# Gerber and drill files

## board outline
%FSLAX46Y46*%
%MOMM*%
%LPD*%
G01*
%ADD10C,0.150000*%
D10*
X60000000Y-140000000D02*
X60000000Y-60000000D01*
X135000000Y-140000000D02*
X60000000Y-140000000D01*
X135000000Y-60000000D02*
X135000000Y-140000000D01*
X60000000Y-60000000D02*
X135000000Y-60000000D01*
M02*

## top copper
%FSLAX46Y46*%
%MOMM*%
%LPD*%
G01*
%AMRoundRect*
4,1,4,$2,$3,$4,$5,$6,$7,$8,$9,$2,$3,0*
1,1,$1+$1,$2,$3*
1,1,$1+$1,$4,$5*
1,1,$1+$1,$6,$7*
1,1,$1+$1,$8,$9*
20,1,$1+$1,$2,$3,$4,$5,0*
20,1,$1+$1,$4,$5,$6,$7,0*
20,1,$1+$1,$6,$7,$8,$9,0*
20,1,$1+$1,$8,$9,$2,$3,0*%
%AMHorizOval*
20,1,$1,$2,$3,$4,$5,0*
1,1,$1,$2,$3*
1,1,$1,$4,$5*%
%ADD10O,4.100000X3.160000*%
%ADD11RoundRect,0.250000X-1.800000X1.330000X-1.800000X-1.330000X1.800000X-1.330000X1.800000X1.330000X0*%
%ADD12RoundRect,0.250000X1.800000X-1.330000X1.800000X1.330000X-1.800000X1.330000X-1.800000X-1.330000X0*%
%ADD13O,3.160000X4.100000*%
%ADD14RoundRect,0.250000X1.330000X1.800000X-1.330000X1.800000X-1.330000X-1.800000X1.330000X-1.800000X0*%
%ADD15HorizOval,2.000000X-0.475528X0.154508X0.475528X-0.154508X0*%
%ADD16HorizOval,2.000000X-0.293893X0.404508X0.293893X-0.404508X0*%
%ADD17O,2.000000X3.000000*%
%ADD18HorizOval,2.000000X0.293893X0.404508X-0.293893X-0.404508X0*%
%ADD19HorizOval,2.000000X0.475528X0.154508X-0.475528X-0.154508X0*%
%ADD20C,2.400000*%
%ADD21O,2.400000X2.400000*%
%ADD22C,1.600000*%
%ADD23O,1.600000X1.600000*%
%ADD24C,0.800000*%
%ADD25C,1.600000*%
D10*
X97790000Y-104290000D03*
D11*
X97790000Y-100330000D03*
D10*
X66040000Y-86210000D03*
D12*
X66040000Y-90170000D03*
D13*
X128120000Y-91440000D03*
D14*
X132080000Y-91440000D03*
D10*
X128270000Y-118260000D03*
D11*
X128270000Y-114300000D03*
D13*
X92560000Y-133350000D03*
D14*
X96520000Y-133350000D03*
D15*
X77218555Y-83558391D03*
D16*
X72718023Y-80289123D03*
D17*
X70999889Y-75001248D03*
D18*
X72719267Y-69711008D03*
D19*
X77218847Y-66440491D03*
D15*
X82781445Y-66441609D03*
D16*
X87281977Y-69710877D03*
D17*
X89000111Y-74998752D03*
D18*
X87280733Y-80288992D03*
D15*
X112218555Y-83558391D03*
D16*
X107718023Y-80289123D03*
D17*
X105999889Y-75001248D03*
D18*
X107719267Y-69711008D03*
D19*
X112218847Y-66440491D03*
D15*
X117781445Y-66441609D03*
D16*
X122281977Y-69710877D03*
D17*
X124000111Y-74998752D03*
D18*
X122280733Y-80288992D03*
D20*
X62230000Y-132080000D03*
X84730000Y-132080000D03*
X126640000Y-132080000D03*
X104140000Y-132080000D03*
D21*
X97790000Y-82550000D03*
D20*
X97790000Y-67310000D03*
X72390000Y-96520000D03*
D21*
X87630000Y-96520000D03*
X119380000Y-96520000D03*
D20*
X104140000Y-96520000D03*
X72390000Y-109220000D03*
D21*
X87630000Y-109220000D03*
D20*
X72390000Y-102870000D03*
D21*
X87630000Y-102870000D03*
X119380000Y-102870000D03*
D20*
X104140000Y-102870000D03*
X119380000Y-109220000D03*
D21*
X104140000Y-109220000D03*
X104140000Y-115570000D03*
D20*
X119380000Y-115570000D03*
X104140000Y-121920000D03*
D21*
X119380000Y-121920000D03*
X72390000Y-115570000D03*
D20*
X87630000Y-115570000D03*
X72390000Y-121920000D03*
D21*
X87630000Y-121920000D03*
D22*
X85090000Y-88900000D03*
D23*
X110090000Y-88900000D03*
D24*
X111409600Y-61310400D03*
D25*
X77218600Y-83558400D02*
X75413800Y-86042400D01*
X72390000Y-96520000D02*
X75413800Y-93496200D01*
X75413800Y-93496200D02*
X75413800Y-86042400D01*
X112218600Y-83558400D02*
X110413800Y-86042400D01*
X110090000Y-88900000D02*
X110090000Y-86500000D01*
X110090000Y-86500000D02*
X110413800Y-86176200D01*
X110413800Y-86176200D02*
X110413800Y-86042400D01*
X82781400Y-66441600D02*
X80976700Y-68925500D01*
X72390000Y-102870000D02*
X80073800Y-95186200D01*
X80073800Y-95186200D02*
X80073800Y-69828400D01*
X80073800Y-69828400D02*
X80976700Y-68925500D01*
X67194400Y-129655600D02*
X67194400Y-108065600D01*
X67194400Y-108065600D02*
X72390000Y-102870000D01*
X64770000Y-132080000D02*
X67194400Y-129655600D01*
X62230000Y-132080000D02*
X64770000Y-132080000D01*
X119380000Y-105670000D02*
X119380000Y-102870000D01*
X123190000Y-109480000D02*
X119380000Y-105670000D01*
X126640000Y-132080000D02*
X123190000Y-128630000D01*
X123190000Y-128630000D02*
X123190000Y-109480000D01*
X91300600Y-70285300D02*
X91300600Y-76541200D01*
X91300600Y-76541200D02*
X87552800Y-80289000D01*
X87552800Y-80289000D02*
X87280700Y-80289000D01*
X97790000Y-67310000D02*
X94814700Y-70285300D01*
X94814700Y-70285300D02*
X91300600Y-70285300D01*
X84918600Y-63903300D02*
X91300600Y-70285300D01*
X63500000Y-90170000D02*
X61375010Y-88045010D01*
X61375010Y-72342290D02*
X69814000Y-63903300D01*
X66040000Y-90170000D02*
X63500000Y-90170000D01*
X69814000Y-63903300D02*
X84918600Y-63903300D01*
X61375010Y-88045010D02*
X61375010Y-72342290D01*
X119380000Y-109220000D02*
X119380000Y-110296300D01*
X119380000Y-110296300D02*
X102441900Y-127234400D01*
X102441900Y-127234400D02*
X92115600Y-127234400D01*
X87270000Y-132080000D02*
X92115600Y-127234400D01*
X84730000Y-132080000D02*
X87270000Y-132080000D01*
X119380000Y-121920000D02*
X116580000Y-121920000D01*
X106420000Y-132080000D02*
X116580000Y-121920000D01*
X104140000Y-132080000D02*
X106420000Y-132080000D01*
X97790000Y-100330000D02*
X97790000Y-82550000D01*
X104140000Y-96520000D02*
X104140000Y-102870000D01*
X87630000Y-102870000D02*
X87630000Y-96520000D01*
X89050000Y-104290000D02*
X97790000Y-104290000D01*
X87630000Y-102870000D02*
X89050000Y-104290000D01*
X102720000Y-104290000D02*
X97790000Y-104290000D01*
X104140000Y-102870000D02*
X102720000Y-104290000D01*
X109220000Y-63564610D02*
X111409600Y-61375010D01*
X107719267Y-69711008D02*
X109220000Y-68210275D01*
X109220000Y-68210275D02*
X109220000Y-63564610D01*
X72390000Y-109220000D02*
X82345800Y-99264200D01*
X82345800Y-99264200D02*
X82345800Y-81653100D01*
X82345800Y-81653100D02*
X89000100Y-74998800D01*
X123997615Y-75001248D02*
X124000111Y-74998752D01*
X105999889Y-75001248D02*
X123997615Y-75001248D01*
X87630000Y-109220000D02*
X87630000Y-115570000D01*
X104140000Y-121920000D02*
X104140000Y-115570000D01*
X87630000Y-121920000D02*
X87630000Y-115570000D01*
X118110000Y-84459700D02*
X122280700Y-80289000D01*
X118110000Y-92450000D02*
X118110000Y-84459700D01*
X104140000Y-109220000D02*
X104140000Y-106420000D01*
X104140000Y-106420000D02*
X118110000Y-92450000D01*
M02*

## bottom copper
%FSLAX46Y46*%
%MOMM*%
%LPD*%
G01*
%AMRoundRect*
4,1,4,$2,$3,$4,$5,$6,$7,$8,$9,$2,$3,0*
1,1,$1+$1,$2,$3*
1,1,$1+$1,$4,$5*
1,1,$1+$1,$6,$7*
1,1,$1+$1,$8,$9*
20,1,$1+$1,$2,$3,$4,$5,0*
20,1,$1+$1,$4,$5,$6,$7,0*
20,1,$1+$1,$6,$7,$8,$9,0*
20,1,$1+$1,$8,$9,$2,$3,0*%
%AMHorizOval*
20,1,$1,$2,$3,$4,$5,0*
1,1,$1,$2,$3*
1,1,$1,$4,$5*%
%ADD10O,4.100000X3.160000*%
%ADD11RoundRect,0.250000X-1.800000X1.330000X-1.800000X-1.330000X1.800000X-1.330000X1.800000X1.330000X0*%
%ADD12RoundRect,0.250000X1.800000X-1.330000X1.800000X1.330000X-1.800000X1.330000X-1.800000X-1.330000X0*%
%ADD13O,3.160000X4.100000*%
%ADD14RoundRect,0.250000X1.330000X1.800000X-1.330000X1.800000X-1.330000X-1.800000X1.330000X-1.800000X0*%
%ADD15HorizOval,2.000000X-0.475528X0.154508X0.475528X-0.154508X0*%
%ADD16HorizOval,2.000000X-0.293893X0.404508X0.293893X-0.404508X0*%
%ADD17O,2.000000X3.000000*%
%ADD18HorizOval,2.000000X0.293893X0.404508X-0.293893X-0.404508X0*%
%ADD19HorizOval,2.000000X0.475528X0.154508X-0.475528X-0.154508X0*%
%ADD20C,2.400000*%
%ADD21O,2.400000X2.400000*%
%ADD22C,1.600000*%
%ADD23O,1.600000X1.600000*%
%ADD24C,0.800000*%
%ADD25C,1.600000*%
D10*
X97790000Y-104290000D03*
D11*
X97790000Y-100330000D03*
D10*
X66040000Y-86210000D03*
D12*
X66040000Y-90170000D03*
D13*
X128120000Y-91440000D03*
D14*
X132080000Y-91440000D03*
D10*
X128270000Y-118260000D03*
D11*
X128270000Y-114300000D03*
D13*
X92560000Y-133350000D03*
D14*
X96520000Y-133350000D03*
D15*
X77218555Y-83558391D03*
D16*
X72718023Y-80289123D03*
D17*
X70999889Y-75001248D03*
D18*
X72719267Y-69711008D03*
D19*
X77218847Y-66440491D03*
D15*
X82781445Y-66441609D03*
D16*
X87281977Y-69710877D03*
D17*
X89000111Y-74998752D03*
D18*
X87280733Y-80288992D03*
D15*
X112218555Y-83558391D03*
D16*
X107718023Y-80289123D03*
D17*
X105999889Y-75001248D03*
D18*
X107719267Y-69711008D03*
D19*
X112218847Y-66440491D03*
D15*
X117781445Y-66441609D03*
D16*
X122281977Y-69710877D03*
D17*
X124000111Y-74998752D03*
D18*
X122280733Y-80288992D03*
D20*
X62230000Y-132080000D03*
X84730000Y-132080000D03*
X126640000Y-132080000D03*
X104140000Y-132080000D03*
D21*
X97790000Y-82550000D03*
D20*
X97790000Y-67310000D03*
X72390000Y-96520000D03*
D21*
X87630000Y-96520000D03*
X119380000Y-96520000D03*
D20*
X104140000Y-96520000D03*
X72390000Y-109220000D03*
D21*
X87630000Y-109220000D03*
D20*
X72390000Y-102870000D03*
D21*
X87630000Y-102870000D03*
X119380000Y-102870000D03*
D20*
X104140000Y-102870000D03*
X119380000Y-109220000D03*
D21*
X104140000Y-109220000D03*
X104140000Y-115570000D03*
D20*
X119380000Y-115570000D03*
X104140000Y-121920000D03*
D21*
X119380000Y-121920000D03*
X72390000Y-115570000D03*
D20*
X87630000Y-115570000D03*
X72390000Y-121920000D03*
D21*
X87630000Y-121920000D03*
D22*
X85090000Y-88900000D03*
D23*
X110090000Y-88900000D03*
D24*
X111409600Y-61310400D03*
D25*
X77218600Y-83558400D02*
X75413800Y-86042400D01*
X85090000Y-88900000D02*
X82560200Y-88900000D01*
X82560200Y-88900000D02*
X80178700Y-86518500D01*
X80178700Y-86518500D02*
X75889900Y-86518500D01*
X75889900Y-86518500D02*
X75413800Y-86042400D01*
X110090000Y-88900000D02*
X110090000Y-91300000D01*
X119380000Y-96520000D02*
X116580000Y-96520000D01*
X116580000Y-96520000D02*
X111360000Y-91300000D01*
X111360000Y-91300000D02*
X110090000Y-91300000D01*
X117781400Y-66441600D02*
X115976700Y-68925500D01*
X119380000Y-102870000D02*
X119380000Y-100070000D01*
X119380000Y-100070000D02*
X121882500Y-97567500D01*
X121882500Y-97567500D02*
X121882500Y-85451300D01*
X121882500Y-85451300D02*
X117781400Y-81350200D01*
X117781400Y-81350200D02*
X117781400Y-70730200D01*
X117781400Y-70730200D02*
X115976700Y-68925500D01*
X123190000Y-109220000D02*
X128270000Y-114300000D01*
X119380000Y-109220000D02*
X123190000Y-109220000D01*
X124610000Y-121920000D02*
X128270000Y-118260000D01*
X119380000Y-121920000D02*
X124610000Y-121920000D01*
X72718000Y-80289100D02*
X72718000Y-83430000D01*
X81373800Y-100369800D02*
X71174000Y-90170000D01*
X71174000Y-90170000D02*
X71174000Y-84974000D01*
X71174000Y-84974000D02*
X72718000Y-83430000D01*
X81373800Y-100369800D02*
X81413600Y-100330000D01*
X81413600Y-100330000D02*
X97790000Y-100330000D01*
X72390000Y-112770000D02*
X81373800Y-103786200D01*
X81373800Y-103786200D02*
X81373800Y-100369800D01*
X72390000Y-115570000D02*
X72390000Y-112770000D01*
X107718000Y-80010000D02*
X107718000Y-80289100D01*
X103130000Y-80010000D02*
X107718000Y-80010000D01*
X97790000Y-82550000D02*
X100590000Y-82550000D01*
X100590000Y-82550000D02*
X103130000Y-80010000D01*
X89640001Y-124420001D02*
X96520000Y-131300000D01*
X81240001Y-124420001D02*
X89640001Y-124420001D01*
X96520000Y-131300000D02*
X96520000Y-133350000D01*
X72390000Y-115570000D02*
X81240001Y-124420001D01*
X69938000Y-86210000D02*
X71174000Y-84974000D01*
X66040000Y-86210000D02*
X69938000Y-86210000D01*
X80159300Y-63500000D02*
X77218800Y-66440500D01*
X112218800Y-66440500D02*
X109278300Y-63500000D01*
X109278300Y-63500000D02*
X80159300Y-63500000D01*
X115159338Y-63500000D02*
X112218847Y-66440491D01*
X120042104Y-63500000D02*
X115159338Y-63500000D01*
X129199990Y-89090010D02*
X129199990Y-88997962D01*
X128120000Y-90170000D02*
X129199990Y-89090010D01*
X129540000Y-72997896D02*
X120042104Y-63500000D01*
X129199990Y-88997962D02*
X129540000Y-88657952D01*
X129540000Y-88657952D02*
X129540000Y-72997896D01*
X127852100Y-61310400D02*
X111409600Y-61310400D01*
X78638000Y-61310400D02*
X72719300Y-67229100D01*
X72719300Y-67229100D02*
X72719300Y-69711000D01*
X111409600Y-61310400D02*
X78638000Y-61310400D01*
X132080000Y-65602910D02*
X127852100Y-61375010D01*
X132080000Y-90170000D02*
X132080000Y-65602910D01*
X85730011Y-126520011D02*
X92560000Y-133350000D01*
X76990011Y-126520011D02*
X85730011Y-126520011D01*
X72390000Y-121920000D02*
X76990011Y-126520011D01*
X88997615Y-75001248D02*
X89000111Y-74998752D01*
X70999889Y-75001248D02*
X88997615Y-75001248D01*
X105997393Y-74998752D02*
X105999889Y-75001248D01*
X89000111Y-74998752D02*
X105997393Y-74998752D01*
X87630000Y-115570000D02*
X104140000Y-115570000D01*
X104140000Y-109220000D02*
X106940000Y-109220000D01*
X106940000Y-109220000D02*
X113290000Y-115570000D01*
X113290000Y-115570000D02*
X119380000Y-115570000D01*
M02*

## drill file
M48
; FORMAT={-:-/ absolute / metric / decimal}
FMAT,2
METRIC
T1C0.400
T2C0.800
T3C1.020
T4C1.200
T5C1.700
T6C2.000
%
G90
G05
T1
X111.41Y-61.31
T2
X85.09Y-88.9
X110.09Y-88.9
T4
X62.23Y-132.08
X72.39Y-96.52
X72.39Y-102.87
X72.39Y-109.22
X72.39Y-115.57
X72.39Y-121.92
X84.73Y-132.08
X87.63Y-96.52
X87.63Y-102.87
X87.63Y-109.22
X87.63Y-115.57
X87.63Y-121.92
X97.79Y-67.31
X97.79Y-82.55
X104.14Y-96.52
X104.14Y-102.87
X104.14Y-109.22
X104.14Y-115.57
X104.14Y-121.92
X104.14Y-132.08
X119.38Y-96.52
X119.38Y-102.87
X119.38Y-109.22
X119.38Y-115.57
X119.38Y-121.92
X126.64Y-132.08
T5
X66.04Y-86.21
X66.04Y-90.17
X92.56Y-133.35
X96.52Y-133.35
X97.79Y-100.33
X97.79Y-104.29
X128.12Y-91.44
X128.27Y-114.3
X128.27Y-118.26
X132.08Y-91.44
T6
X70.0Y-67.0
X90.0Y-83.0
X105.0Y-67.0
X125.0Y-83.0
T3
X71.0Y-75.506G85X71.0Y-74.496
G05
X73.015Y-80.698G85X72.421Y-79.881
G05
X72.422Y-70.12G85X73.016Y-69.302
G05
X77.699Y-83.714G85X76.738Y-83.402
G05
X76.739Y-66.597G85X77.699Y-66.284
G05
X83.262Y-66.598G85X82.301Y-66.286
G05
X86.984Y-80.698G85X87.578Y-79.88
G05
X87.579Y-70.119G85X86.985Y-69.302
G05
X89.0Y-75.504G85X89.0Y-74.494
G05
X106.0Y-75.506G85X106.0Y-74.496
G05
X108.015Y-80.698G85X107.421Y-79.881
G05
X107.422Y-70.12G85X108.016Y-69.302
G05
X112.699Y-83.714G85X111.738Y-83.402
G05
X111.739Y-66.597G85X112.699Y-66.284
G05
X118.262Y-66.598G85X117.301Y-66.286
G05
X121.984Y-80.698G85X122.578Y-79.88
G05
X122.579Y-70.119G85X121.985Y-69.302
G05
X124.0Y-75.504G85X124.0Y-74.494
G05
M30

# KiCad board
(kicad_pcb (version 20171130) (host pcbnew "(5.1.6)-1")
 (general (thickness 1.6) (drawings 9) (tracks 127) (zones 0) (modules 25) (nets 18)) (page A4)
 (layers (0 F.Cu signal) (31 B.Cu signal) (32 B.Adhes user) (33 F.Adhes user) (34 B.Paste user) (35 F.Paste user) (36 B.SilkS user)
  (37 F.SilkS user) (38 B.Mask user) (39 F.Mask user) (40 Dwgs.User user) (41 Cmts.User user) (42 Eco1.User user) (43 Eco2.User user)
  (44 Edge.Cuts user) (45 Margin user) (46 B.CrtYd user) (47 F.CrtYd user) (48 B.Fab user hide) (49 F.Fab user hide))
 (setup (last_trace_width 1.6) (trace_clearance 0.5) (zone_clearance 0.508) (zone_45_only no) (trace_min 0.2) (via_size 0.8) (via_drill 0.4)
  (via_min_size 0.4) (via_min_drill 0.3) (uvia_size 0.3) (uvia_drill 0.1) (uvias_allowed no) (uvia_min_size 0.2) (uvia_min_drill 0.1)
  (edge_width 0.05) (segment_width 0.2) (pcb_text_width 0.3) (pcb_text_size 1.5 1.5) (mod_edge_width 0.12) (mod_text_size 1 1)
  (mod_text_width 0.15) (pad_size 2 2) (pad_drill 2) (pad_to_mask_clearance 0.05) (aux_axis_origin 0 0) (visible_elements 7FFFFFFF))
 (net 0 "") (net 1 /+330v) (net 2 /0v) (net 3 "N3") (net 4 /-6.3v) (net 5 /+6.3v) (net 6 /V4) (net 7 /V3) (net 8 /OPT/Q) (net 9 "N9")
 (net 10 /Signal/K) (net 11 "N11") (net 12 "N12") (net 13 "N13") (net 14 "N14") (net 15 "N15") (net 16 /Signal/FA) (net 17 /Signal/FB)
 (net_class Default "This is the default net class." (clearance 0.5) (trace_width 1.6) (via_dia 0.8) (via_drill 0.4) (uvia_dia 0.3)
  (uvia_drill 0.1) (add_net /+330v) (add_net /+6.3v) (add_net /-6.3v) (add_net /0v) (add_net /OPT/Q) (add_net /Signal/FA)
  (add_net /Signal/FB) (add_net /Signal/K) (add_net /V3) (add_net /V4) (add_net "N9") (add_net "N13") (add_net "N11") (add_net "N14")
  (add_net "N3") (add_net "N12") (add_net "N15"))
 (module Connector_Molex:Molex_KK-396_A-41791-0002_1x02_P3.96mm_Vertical (layer F.Cu) (at 97.79 100.33 270)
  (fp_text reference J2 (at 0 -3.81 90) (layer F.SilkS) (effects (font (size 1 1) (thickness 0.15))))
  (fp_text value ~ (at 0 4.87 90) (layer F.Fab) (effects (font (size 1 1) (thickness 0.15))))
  (pad 2 thru_hole oval (at 3.96 0 270) (size 3.16 4.1) (drill 1.7) (layers *.Cu *.Mask) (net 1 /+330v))
  (pad 1 thru_hole roundrect (at 0 0 270) (size 3.16 4.1) (drill 1.7) (layers *.Cu *.Mask) (roundrect_rratio 0.079114) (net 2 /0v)))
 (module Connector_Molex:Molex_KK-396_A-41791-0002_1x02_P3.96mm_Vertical (layer F.Cu) (at 66.04 90.17 90)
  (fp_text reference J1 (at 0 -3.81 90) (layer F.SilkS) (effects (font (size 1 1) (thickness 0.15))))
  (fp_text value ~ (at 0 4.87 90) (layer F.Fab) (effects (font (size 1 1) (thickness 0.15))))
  (pad 2 thru_hole oval (at 3.96 0 90) (size 3.16 4.1) (drill 1.7) (layers *.Cu *.Mask) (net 2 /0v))
  (pad 1 thru_hole roundrect (at 0 0 90) (size 3.16 4.1) (drill 1.7) (layers *.Cu *.Mask) (roundrect_rratio 0.079114) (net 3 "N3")))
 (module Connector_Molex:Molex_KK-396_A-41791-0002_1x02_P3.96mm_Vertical (layer F.Cu) (at 132.08 91.44 180)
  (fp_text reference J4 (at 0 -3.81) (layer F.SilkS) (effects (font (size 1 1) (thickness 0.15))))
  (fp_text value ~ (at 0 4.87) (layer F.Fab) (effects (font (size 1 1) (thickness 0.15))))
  (pad 2 thru_hole oval (at 3.96 0 180) (size 3.16 4.1) (drill 1.7) (layers *.Cu *.Mask) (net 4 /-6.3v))
  (pad 1 thru_hole roundrect (at 0 0 180) (size 3.16 4.1) (drill 1.7) (layers *.Cu *.Mask) (roundrect_rratio 0.079114) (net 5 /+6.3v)))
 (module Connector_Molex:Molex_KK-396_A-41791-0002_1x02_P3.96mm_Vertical (layer F.Cu) (at 128.27 114.3 270)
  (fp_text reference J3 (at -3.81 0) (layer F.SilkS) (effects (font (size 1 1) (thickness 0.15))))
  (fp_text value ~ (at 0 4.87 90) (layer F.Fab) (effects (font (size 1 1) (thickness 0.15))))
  (pad 2 thru_hole oval (at 3.96 0 270) (size 3.16 4.1) (drill 1.7) (layers *.Cu *.Mask) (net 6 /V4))
  (pad 1 thru_hole roundrect (at 0 0 270) (size 3.16 4.1) (drill 1.7) (layers *.Cu *.Mask) (roundrect_rratio 0.079114) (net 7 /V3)))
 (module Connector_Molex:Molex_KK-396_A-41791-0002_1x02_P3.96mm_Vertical (layer F.Cu) (at 96.52 133.35 180)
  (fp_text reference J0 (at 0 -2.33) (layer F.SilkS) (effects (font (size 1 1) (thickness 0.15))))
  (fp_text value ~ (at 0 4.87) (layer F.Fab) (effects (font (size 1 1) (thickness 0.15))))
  (pad 2 thru_hole oval (at 3.96 0 180) (size 3.16 4.1) (drill 1.7) (layers *.Cu *.Mask) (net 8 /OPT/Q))
  (pad 1 thru_hole roundrect (at 0 0 180) (size 3.16 4.1) (drill 1.7) (layers *.Cu *.Mask) (roundrect_rratio 0.079114) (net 2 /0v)))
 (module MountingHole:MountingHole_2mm (layer F.Cu) (at 90 83)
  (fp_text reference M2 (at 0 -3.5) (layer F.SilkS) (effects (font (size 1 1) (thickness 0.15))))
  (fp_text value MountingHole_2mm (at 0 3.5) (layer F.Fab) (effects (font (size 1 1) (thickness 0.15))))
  (pad "" np_thru_hole circle (at 0 0) (size 2 2) (drill 2) (layers *.Cu *.Mask)))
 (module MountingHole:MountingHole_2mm (layer F.Cu) (at 70 67)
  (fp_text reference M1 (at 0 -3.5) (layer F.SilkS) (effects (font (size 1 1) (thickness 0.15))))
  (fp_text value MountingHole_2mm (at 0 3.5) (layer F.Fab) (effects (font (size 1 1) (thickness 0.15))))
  (pad "" np_thru_hole circle (at 0 0) (size 2 2) (drill 2) (layers *.Cu *.Mask)))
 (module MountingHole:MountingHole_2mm (layer F.Cu) (at 105 67)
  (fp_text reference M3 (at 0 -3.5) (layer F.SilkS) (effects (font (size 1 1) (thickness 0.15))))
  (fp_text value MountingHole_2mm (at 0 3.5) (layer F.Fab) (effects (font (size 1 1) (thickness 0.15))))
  (pad "" np_thru_hole circle (at 0 0) (size 2 2) (drill 2) (layers *.Cu *.Mask)))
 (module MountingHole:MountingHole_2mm (layer F.Cu) (at 125 83)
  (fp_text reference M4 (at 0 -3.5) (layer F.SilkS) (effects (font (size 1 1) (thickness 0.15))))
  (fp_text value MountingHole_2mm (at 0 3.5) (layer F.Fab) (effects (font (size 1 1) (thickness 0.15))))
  (pad "" np_thru_hole circle (at 0 0) (size 2 2) (drill 2) (layers *.Cu *.Mask)))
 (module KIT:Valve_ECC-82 (layer B.Cu) (at 80 75 198)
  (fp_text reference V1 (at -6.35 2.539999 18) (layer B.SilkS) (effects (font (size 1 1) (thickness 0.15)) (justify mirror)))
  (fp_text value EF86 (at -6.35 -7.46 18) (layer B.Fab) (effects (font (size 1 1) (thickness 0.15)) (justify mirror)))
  (pad 1 thru_hole oval (at 5.29 -7.28 252) (size 2 3) (drill oval 1.02 2.03) (layers *.Cu *.Mask) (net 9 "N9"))
  (pad 2 thru_hole oval (at 8.56 -2.78 216) (size 2 3) (drill oval 1.02 2.03) (layers *.Cu *.Mask) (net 2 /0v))
  (pad 3 thru_hole oval (at 8.56 2.78 180) (size 2 3) (drill oval 1.02 2.03) (layers *.Cu *.Mask) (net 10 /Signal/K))
  (pad 4 thru_hole oval (at 5.29 7.28 144) (size 2 3) (drill oval 1.02 2.03) (layers *.Cu *.Mask) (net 5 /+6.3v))
  (pad 5 thru_hole oval (at 0 9 108) (size 2 3) (drill oval 1.02 2.03) (layers *.Cu *.Mask) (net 4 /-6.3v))
  (pad 6 thru_hole oval (at -5.29 7.28 252) (size 2 3) (drill oval 1.02 2.03) (layers *.Cu *.Mask) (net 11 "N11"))
  (pad 7 thru_hole oval (at -8.56 2.78 216) (size 2 3) (drill oval 1.02 2.03) (layers *.Cu *.Mask) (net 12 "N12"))
  (pad 8 thru_hole oval (at -8.56 -2.78 180) (size 2 3) (drill oval 1.02 2.03) (layers *.Cu *.Mask) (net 10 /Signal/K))
  (pad 9 thru_hole oval (at -5.29 -7.28 144) (size 2 3) (drill oval 1.02 2.03) (layers *.Cu *.Mask) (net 3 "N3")))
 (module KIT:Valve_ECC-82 (layer B.Cu) (at 115 75 198)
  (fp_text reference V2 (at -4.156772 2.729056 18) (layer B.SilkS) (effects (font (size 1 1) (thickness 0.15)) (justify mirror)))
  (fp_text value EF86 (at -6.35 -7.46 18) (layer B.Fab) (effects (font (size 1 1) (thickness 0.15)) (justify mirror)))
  (pad 1 thru_hole oval (at 5.29 -7.28 252) (size 2 3) (drill oval 1.02 2.03) (layers *.Cu *.Mask) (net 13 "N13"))
  (pad 2 thru_hole oval (at 8.56 -2.78 216) (size 2 3) (drill oval 1.02 2.03) (layers *.Cu *.Mask) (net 2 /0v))
  (pad 3 thru_hole oval (at 8.56 2.78 180) (size 2 3) (drill oval 1.02 2.03) (layers *.Cu *.Mask) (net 10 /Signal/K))
  (pad 4 thru_hole oval (at 5.29 7.28 144) (size 2 3) (drill oval 1.02 2.03) (layers *.Cu *.Mask) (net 5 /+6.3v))
  (pad 5 thru_hole oval (at 0 9 108) (size 2 3) (drill oval 1.02 2.03) (layers *.Cu *.Mask) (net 4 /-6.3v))
  (pad 6 thru_hole oval (at -5.29 7.28 252) (size 2 3) (drill oval 1.02 2.03) (layers *.Cu *.Mask) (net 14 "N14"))
  (pad 7 thru_hole oval (at -8.56 2.78 216) (size 2 3) (drill oval 1.02 2.03) (layers *.Cu *.Mask) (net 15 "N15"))
  (pad 8 thru_hole oval (at -8.56 -2.78 180) (size 2 3) (drill oval 1.02 2.03) (layers *.Cu *.Mask) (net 10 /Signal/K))
  (pad 9 thru_hole oval (at -5.29 -7.28 144) (size 2 3) (drill oval 1.02 2.03) (layers *.Cu *.Mask) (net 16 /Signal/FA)))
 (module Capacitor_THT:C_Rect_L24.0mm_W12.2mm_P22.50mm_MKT (layer F.Cu) (at 62.23 132.08)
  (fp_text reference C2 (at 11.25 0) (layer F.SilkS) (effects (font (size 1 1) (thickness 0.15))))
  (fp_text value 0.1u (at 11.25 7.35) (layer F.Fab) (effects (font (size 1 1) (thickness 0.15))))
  (pad 1 thru_hole circle (at 0 0) (size 2.4 2.4) (drill 1.2) (layers *.Cu *.Mask) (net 11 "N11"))
  (pad 2 thru_hole circle (at 22.5 0) (size 2.4 2.4) (drill 1.2) (layers *.Cu *.Mask) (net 7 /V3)))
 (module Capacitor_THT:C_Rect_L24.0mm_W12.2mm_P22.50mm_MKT (layer F.Cu) (at 104.14 132.08)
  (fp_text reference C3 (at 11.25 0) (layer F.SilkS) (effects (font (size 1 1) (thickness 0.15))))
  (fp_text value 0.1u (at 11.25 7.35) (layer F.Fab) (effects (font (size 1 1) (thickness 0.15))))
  (pad 2 thru_hole circle (at 22.5 0) (size 2.4 2.4) (drill 1.2) (layers *.Cu *.Mask) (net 14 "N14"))
  (pad 1 thru_hole circle (at 0 0) (size 2.4 2.4) (drill 1.2) (layers *.Cu *.Mask) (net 6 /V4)))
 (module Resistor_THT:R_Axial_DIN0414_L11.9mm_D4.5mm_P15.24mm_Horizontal (layer F.Cu) (at 97.79 67.31 270)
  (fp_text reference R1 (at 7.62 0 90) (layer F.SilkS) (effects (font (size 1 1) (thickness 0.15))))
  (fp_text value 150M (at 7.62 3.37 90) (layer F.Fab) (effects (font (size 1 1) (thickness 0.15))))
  (pad 2 thru_hole oval (at 15.24 0 270) (size 2.4 2.4) (drill 1.2) (layers *.Cu *.Mask) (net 2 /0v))
  (pad 1 thru_hole circle (at 0 0 270) (size 2.4 2.4) (drill 1.2) (layers *.Cu *.Mask) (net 3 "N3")))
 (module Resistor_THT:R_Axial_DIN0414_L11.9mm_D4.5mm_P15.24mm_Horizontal (layer F.Cu) (at 72.39 96.52)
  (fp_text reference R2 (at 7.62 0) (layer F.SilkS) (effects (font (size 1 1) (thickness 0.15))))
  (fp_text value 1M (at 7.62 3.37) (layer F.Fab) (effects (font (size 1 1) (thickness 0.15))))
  (pad 1 thru_hole circle (at 0 0) (size 2.4 2.4) (drill 1.2) (layers *.Cu *.Mask) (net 9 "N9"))
  (pad 2 thru_hole oval (at 15.24 0) (size 2.4 2.4) (drill 1.2) (layers *.Cu *.Mask) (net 1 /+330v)))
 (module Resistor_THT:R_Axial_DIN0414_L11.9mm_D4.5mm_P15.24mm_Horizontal (layer F.Cu) (at 104.14 96.52)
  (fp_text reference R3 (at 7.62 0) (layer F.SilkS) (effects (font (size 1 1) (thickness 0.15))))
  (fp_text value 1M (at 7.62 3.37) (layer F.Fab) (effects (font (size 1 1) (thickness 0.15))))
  (pad 2 thru_hole oval (at 15.24 0) (size 2.4 2.4) (drill 1.2) (layers *.Cu *.Mask) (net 13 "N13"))
  (pad 1 thru_hole circle (at 0 0) (size 2.4 2.4) (drill 1.2) (layers *.Cu *.Mask) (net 1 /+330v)))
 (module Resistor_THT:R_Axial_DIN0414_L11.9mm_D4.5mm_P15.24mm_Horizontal (layer F.Cu) (at 72.39 109.22)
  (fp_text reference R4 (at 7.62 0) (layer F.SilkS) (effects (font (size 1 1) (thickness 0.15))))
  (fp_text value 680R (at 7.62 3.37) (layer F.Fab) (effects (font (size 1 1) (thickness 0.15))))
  (pad 1 thru_hole circle (at 0 0) (size 2.4 2.4) (drill 1.2) (layers *.Cu *.Mask) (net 10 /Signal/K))
  (pad 2 thru_hole oval (at 15.24 0) (size 2.4 2.4) (drill 1.2) (layers *.Cu *.Mask) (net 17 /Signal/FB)))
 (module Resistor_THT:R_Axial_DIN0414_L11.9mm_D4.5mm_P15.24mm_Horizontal (layer F.Cu) (at 72.39 102.87)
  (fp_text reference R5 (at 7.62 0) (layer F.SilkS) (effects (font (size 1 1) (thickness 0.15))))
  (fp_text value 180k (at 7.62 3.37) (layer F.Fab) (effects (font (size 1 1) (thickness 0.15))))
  (pad 1 thru_hole circle (at 0 0) (size 2.4 2.4) (drill 1.2) (layers *.Cu *.Mask) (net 11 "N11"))
  (pad 2 thru_hole oval (at 15.24 0) (size 2.4 2.4) (drill 1.2) (layers *.Cu *.Mask) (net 1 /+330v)))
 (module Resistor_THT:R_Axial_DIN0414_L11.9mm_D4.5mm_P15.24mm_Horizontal (layer F.Cu) (at 104.14 102.87)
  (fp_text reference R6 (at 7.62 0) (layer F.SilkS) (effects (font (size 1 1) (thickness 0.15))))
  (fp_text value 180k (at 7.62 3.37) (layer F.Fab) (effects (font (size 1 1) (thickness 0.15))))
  (pad 2 thru_hole oval (at 15.24 0) (size 2.4 2.4) (drill 1.2) (layers *.Cu *.Mask) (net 14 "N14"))
  (pad 1 thru_hole circle (at 0 0) (size 2.4 2.4) (drill 1.2) (layers *.Cu *.Mask) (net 1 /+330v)))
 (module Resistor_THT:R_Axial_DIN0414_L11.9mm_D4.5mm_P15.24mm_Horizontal (layer F.Cu) (at 119.38 109.22 180)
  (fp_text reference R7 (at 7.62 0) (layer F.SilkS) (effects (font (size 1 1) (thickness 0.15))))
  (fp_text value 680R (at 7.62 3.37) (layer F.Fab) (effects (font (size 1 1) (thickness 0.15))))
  (pad 1 thru_hole circle (at 0 0 180) (size 2.4 2.4) (drill 1.2) (layers *.Cu *.Mask) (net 7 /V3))
  (pad 2 thru_hole oval (at 15.24 0 180) (size 2.4 2.4) (drill 1.2) (layers *.Cu *.Mask) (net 16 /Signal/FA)))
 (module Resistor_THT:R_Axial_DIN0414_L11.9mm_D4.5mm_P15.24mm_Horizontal (layer F.Cu) (at 119.38 115.57 180)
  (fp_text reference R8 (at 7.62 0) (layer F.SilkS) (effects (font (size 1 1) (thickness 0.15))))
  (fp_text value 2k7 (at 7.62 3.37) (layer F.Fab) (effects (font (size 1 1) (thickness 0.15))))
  (pad 2 thru_hole oval (at 15.24 0 180) (size 2.4 2.4) (drill 1.2) (layers *.Cu *.Mask) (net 17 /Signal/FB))
  (pad 1 thru_hole circle (at 0 0 180) (size 2.4 2.4) (drill 1.2) (layers *.Cu *.Mask) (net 16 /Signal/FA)))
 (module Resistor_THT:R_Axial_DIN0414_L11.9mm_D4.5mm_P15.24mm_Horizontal (layer F.Cu) (at 104.14 121.92)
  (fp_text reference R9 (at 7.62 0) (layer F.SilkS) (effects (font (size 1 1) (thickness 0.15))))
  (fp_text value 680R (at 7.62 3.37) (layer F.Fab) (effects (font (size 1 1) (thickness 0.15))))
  (pad 1 thru_hole circle (at 0 0) (size 2.4 2.4) (drill 1.2) (layers *.Cu *.Mask) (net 17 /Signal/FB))
  (pad 2 thru_hole oval (at 15.24 0) (size 2.4 2.4) (drill 1.2) (layers *.Cu *.Mask) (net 6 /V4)))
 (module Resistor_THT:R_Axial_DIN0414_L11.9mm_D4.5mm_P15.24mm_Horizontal (layer F.Cu) (at 87.63 115.57 180)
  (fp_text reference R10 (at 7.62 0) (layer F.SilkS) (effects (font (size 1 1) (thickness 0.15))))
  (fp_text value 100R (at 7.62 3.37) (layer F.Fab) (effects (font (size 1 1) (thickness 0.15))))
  (pad 2 thru_hole oval (at 15.24 0 180) (size 2.4 2.4) (drill 1.2) (layers *.Cu *.Mask) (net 2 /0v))
  (pad 1 thru_hole circle (at 0 0 180) (size 2.4 2.4) (drill 1.2) (layers *.Cu *.Mask) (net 17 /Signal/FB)))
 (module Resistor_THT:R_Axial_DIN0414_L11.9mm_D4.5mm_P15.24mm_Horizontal (layer F.Cu) (at 72.39 121.92)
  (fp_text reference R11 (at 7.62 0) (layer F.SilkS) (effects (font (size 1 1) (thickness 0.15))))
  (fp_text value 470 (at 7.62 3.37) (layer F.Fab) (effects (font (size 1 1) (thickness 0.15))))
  (pad 1 thru_hole circle (at 0 0) (size 2.4 2.4) (drill 1.2) (layers *.Cu *.Mask) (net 8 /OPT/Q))
  (pad 2 thru_hole oval (at 15.24 0) (size 2.4 2.4) (drill 1.2) (layers *.Cu *.Mask) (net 17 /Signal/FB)))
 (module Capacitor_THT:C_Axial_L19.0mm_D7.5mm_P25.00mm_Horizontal (layer F.Cu) (at 85.09 88.9)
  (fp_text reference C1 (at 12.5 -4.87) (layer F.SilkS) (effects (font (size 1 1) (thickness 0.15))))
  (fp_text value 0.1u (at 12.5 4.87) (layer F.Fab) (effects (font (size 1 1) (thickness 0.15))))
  (pad 1 thru_hole circle (at 0 0) (size 1.6 1.6) (drill 0.8) (layers *.Cu *.Mask) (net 9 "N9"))
  (pad 2 thru_hole oval (at 25 0) (size 1.6 1.6) (drill 0.8) (layers *.Cu *.Mask) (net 13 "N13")))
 (gr_line (start 60 140) (end 60 60) (layer Edge.Cuts) (width 0.15))
 (gr_line (start 135 140) (end 60 140) (layer Edge.Cuts) (width 0.15))
 (gr_line (start 135 60) (end 135 140) (layer Edge.Cuts) (width 0.15))
 (gr_line (start 60 60) (end 135 60) (layer Edge.Cuts) (width 0.15))
 (segment (start 77.2186 83.5584) (end 75.4138 86.0424) (width 1.6) (layer F.Cu) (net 9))
 (segment (start 72.39 96.52) (end 75.4138 93.4962) (width 1.6) (layer F.Cu) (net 9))
 (segment (start 75.4138 93.4962) (end 75.4138 86.0424) (width 1.6) (layer F.Cu) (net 9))
 (segment (start 77.2186 83.5584) (end 75.4138 86.0424) (width 1.6) (layer B.Cu) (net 9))
 (segment (start 85.09 88.9) (end 82.5602 88.9) (width 1.6) (layer B.Cu) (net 9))
 (segment (start 82.5602 88.9) (end 80.1787 86.5185) (width 1.6) (layer B.Cu) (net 9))
 (segment (start 80.1787 86.5185) (end 75.8899 86.5185) (width 1.6) (layer B.Cu) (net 9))
 (segment (start 75.8899 86.5185) (end 75.4138 86.0424) (width 1.6) (layer B.Cu) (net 9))
 (segment (start 110.09 88.9) (end 110.09 91.3) (width 1.6) (layer B.Cu) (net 13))
 (segment (start 119.38 96.52) (end 116.58 96.52) (width 1.6) (layer B.Cu) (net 13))
 (segment (start 116.58 96.52) (end 111.36 91.3) (width 1.6) (layer B.Cu) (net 13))
 (segment (start 111.36 91.3) (end 110.09 91.3) (width 1.6) (layer B.Cu) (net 13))
 (segment (start 112.2186 83.5584) (end 110.4138 86.0424) (width 1.6) (layer F.Cu) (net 13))
 (segment (start 110.09 88.9) (end 110.09 86.5) (width 1.6) (layer F.Cu) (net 13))
 (segment (start 110.09 86.5) (end 110.4138 86.1762) (width 1.6) (layer F.Cu) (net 13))
 (segment (start 110.4138 86.1762) (end 110.4138 86.0424) (width 1.6) (layer F.Cu) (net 13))
 (segment (start 82.7814 66.4416) (end 80.9767 68.9255) (width 1.6) (layer F.Cu) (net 11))
 (segment (start 72.39 102.87) (end 80.0738 95.1862) (width 1.6) (layer F.Cu) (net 11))
 (segment (start 80.0738 95.1862) (end 80.0738 69.8284) (width 1.6) (layer F.Cu) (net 11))
 (segment (start 80.0738 69.8284) (end 80.9767 68.9255) (width 1.6) (layer F.Cu) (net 11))
 (segment (start 67.1944 129.6556) (end 67.1944 108.0656) (width 1.6) (layer F.Cu) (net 11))
 (segment (start 67.1944 108.0656) (end 72.39 102.87) (width 1.6) (layer F.Cu) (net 11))
 (segment (start 64.77 132.08) (end 67.1944 129.6556) (width 1.6) (layer F.Cu) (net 11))
 (segment (start 62.23 132.08) (end 64.77 132.08) (width 1.6) (layer F.Cu) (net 11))
 (segment (start 117.7814 66.4416) (end 115.9767 68.9255) (width 1.6) (layer B.Cu) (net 14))
 (segment (start 119.38 102.87) (end 119.38 100.07) (width 1.6) (layer B.Cu) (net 14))
 (segment (start 119.38 100.07) (end 121.8825 97.5675) (width 1.6) (layer B.Cu) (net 14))
 (segment (start 121.8825 97.5675) (end 121.8825 85.4513) (width 1.6) (layer B.Cu) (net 14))
 (segment (start 121.8825 85.4513) (end 117.7814 81.3502) (width 1.6) (layer B.Cu) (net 14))
 (segment (start 117.7814 81.3502) (end 117.7814 70.7302) (width 1.6) (layer B.Cu) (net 14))
 (segment (start 117.7814 70.7302) (end 115.9767 68.9255) (width 1.6) (layer B.Cu) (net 14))
 (segment (start 119.38 105.67) (end 119.38 102.87) (width 1.6) (layer F.Cu) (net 14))
 (segment (start 123.19 109.48) (end 119.38 105.67) (width 1.6) (layer F.Cu) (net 14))
 (segment (start 126.64 132.08) (end 123.19 128.63) (width 1.6) (layer F.Cu) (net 14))
 (segment (start 123.19 128.63) (end 123.19 109.48) (width 1.6) (layer F.Cu) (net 14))
 (segment (start 91.3006 70.2853) (end 91.3006 76.5412) (width 1.6) (layer F.Cu) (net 3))
 (segment (start 91.3006 76.5412) (end 87.5528 80.289) (width 1.6) (layer F.Cu) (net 3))
 (segment (start 87.5528 80.289) (end 87.2807 80.289) (width 1.6) (layer F.Cu) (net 3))
 (segment (start 97.79 67.31) (end 94.8147 70.2853) (width 1.6) (layer F.Cu) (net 3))
 (segment (start 94.8147 70.2853) (end 91.3006 70.2853) (width 1.6) (layer F.Cu) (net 3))
 (segment (start 84.9186 63.9033) (end 91.3006 70.2853) (width 1.6) (layer F.Cu) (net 3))
 (segment (start 63.5 90.17) (end 61.37501 88.04501) (width 1.6) (layer F.Cu) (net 3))
 (segment (start 61.37501 72.34229) (end 69.814 63.9033) (width 1.6) (layer F.Cu) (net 3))
 (segment (start 66.04 90.17) (end 63.5 90.17) (width 1.6) (layer F.Cu) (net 3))
 (segment (start 69.814 63.9033) (end 84.9186 63.9033) (width 1.6) (layer F.Cu) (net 3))
 (segment (start 61.37501 88.04501) (end 61.37501 72.34229) (width 1.6) (layer F.Cu) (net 3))
 (segment (start 119.38 109.22) (end 119.38 110.2963) (width 1.6) (layer F.Cu) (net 7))
 (segment (start 119.38 110.2963) (end 102.4419 127.2344) (width 1.6) (layer F.Cu) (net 7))
 (segment (start 102.4419 127.2344) (end 92.1156 127.2344) (width 1.6) (layer F.Cu) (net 7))
 (segment (start 87.27 132.08) (end 92.1156 127.2344) (width 1.6) (layer F.Cu) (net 7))
 (segment (start 84.73 132.08) (end 87.27 132.08) (width 1.6) (layer F.Cu) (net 7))
 (segment (start 123.19 109.22) (end 128.27 114.3) (width 1.6) (layer B.Cu) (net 7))
 (segment (start 119.38 109.22) (end 123.19 109.22) (width 1.6) (layer B.Cu) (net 7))
 (segment (start 119.38 121.92) (end 116.58 121.92) (width 1.6) (layer F.Cu) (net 6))
 (segment (start 106.42 132.08) (end 116.58 121.92) (width 1.6) (layer F.Cu) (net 6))
 (segment (start 104.14 132.08) (end 106.42 132.08) (width 1.6) (layer F.Cu) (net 6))
 (segment (start 124.61 121.92) (end 128.27 118.26) (width 1.6) (layer B.Cu) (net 6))
 (segment (start 119.38 121.92) (end 124.61 121.92) (width 1.6) (layer B.Cu) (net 6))
 (segment (start 72.718 80.2891) (end 72.718 83.43) (width 1.6) (layer B.Cu) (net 2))
 (segment (start 81.3738 100.3698) (end 71.174 90.17) (width 1.6) (layer B.Cu) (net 2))
 (segment (start 71.174 90.17) (end 71.174 84.974) (width 1.6) (layer B.Cu) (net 2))
 (segment (start 71.174 84.974) (end 72.718 83.43) (width 1.6) (layer B.Cu) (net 2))
 (segment (start 81.3738 100.3698) (end 81.4136 100.33) (width 1.6) (layer B.Cu) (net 2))
 (segment (start 81.4136 100.33) (end 97.79 100.33) (width 1.6) (layer B.Cu) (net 2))
 (segment (start 72.39 112.77) (end 81.3738 103.7862) (width 1.6) (layer B.Cu) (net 2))
 (segment (start 81.3738 103.7862) (end 81.3738 100.3698) (width 1.6) (layer B.Cu) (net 2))
 (segment (start 72.39 115.57) (end 72.39 112.77) (width 1.6) (layer B.Cu) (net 2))
 (segment (start 97.79 100.33) (end 97.79 82.55) (width 1.6) (layer F.Cu) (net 2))
 (segment (start 107.718 80.01) (end 107.718 80.2891) (width 1.6) (layer B.Cu) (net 2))
 (segment (start 103.13 80.01) (end 107.718 80.01) (width 1.6) (layer B.Cu) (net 2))
 (segment (start 97.79 82.55) (end 100.59 82.55) (width 1.6) (layer B.Cu) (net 2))
 (segment (start 100.59 82.55) (end 103.13 80.01) (width 1.6) (layer B.Cu) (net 2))
 (segment (start 89.640001 124.420001) (end 96.52 131.3) (width 1.6) (layer B.Cu) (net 2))
 (segment (start 81.240001 124.420001) (end 89.640001 124.420001) (width 1.6) (layer B.Cu) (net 2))
 (segment (start 96.52 131.3) (end 96.52 133.35) (width 1.6) (layer B.Cu) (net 2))
 (segment (start 72.39 115.57) (end 81.240001 124.420001) (width 1.6) (layer B.Cu) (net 2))
 (segment (start 69.938 86.21) (end 71.174 84.974) (width 1.6) (layer B.Cu) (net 2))
 (segment (start 66.04 86.21) (end 69.938 86.21) (width 1.6) (layer B.Cu) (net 2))
 (segment (start 104.14 96.52) (end 104.14 102.87) (width 1.6) (layer F.Cu) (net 1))
 (segment (start 87.63 102.87) (end 87.63 96.52) (width 1.6) (layer F.Cu) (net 1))
 (segment (start 89.05 104.29) (end 97.79 104.29) (width 1.6) (layer F.Cu) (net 1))
 (segment (start 87.63 102.87) (end 89.05 104.29) (width 1.6) (layer F.Cu) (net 1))
 (segment (start 102.72 104.29) (end 97.79 104.29) (width 1.6) (layer F.Cu) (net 1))
 (segment (start 104.14 102.87) (end 102.72 104.29) (width 1.6) (layer F.Cu) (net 1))
 (segment (start 80.1593 63.5) (end 77.2188 66.4405) (width 1.6) (layer B.Cu) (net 4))
 (segment (start 112.2188 66.4405) (end 109.2783 63.5) (width 1.6) (layer B.Cu) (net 4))
 (segment (start 109.2783 63.5) (end 80.1593 63.5) (width 1.6) (layer B.Cu) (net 4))
 (segment (start 115.159338 63.5) (end 112.218847 66.440491) (width 1.6) (layer B.Cu) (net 4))
 (segment (start 120.042104 63.5) (end 115.159338 63.5) (width 1.6) (layer B.Cu) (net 4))
 (segment (start 129.19999 89.09001) (end 129.19999 88.997962) (width 1.6) (layer B.Cu) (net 4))
 (segment (start 128.12 90.17) (end 129.19999 89.09001) (width 1.6) (layer B.Cu) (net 4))
 (segment (start 129.54 72.997896) (end 120.042104 63.5) (width 1.6) (layer B.Cu) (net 4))
 (segment (start 129.19999 88.997962) (end 129.54 88.657952) (width 1.6) (layer B.Cu) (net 4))
 (segment (start 129.54 88.657952) (end 129.54 72.997896) (width 1.6) (layer B.Cu) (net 4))
 (segment (start 127.8521 61.3104) (end 111.4096 61.3104) (width 1.6) (layer B.Cu) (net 5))
 (segment (start 78.638 61.3104) (end 72.7193 67.2291) (width 1.6) (layer B.Cu) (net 5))
 (segment (start 72.7193 67.2291) (end 72.7193 69.711) (width 1.6) (layer B.Cu) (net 5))
 (segment (start 111.4096 61.3104) (end 78.638 61.3104) (width 1.6) (layer B.Cu) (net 5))
 (via (at 111.4096 61.3104) (size 0.8) (drill 0.4) (layers F.Cu B.Cu) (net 5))
 (segment (start 132.08 65.60291) (end 127.8521 61.37501) (width 1.6) (layer B.Cu) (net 5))
 (segment (start 132.08 90.17) (end 132.08 65.60291) (width 1.6) (layer B.Cu) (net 5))
 (segment (start 109.22 63.56461) (end 111.4096 61.37501) (width 1.6) (layer F.Cu) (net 5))
 (segment (start 107.719267 69.711008) (end 109.22 68.210275) (width 1.6) (layer F.Cu) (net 5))
 (segment (start 109.22 68.210275) (end 109.22 63.56461) (width 1.6) (layer F.Cu) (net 5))
 (segment (start 85.730011 126.520011) (end 92.56 133.35) (width 1.6) (layer B.Cu) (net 8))
 (segment (start 76.990011 126.520011) (end 85.730011 126.520011) (width 1.6) (layer B.Cu) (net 8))
 (segment (start 72.39 121.92) (end 76.990011 126.520011) (width 1.6) (layer B.Cu) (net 8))
 (segment (start 72.39 109.22) (end 82.3458 99.2642) (width 1.6) (layer F.Cu) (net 10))
 (segment (start 82.3458 99.2642) (end 82.3458 81.6531) (width 1.6) (layer F.Cu) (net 10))
 (segment (start 82.3458 81.6531) (end 89.0001 74.9988) (width 1.6) (layer F.Cu) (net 10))
 (segment (start 88.997615 75.001248) (end 89.000111 74.998752) (width 1.6) (layer B.Cu) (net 10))
 (segment (start 70.999889 75.001248) (end 88.997615 75.001248) (width 1.6) (layer B.Cu) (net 10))
 (segment (start 105.997393 74.998752) (end 105.999889 75.001248) (width 1.6) (layer B.Cu) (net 10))
 (segment (start 89.000111 74.998752) (end 105.997393 74.998752) (width 1.6) (layer B.Cu) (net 10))
 (segment (start 123.997615 75.001248) (end 124.000111 74.998752) (width 1.6) (layer F.Cu) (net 10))
 (segment (start 105.999889 75.001248) (end 123.997615 75.001248) (width 1.6) (layer F.Cu) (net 10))
 (segment (start 87.63 115.57) (end 104.14 115.57) (width 1.6) (layer B.Cu) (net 17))
 (segment (start 87.63 109.22) (end 87.63 115.57) (width 1.6) (layer F.Cu) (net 17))
 (segment (start 104.14 121.92) (end 104.14 115.57) (width 1.6) (layer F.Cu) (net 17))
 (segment (start 87.63 121.92) (end 87.63 115.57) (width 1.6) (layer F.Cu) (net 17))
 (segment (start 104.14 109.22) (end 106.94 109.22) (width 1.6) (layer B.Cu) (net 16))
 (segment (start 106.94 109.22) (end 113.29 115.57) (width 1.6) (layer B.Cu) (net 16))
 (segment (start 113.29 115.57) (end 119.38 115.57) (width 1.6) (layer B.Cu) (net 16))
 (segment (start 118.11 84.4597) (end 122.2807 80.289) (width 1.6) (layer F.Cu) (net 16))
 (segment (start 118.11 92.45) (end 118.11 84.4597) (width 1.6) (layer F.Cu) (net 16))
 (segment (start 104.14 109.22) (end 104.14 106.42) (width 1.6) (layer F.Cu) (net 16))
 (segment (start 104.14 106.42) (end 118.11 92.45) (width 1.6) (layer F.Cu) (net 16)))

